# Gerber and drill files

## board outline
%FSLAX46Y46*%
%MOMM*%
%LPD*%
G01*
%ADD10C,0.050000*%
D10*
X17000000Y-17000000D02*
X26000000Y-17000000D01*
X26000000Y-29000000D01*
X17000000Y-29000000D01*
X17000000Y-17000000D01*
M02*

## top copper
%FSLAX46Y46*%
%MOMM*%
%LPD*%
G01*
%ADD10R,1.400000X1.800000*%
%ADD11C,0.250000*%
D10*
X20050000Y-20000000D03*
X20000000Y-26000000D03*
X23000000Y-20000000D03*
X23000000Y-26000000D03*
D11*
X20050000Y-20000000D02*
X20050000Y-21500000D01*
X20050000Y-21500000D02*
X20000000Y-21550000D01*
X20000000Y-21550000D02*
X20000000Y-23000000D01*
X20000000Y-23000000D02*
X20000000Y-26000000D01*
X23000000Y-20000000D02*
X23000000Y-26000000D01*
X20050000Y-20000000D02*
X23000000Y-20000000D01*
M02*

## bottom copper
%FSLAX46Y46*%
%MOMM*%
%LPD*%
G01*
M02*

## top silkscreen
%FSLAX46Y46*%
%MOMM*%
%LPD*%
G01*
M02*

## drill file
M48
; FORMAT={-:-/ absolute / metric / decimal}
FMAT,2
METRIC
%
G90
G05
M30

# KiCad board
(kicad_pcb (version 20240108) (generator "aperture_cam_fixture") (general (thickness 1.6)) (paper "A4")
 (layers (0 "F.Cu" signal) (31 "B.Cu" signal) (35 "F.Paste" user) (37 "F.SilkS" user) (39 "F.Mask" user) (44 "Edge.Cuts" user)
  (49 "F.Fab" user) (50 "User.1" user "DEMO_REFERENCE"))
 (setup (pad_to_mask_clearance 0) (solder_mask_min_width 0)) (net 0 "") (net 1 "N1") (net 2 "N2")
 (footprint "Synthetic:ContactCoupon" (layer "F.Cu") (at 20 20)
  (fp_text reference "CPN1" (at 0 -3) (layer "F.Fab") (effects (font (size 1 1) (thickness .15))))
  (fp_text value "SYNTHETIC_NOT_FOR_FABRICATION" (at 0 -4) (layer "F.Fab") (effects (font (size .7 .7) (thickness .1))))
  (pad "1" smd rect (at 0.050000 0.000000) (size 1.4 1.8) (layers "F.Cu") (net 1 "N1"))
  (pad "2" smd rect (at 0.000000 6.000000) (size 1.4 1.8) (layers "F.Cu") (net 1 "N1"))
  (pad "3" smd rect (at 3.000000 0.000000) (size 1.4 1.8) (layers "F.Cu") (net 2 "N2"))
  (pad "4" smd rect (at 3.000000 6.000000) (size 1.4 1.8) (layers "F.Cu") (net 2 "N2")))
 (segment (start 20.050000 20.000000) (end 20.050000 21.500000) (width 0.25) (layer "F.Cu") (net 1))
 (segment (start 20.050000 21.500000) (end 20.000000 21.550000) (width 0.25) (layer "F.Cu") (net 1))
 (segment (start 20.000000 21.550000) (end 20.000000 23.000000) (width 0.25) (layer "F.Cu") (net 1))
 (segment (start 20.000000 23.000000) (end 20.000000 26.000000) (width 0.25) (layer "F.Cu") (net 1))
 (segment (start 23.000000 20.000000) (end 23.000000 26.000000) (width 0.25) (layer "F.Cu") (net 2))
 (segment (start 20.050000 20.000000) (end 23.000000 20.000000) (width 0.25) (layer "F.Cu") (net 1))
 (gr_rect locked (start 17.0 17.0) (end 26.0 29.0) (stroke (width .05) (type default)) (fill none) (layer "Edge.Cuts")))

